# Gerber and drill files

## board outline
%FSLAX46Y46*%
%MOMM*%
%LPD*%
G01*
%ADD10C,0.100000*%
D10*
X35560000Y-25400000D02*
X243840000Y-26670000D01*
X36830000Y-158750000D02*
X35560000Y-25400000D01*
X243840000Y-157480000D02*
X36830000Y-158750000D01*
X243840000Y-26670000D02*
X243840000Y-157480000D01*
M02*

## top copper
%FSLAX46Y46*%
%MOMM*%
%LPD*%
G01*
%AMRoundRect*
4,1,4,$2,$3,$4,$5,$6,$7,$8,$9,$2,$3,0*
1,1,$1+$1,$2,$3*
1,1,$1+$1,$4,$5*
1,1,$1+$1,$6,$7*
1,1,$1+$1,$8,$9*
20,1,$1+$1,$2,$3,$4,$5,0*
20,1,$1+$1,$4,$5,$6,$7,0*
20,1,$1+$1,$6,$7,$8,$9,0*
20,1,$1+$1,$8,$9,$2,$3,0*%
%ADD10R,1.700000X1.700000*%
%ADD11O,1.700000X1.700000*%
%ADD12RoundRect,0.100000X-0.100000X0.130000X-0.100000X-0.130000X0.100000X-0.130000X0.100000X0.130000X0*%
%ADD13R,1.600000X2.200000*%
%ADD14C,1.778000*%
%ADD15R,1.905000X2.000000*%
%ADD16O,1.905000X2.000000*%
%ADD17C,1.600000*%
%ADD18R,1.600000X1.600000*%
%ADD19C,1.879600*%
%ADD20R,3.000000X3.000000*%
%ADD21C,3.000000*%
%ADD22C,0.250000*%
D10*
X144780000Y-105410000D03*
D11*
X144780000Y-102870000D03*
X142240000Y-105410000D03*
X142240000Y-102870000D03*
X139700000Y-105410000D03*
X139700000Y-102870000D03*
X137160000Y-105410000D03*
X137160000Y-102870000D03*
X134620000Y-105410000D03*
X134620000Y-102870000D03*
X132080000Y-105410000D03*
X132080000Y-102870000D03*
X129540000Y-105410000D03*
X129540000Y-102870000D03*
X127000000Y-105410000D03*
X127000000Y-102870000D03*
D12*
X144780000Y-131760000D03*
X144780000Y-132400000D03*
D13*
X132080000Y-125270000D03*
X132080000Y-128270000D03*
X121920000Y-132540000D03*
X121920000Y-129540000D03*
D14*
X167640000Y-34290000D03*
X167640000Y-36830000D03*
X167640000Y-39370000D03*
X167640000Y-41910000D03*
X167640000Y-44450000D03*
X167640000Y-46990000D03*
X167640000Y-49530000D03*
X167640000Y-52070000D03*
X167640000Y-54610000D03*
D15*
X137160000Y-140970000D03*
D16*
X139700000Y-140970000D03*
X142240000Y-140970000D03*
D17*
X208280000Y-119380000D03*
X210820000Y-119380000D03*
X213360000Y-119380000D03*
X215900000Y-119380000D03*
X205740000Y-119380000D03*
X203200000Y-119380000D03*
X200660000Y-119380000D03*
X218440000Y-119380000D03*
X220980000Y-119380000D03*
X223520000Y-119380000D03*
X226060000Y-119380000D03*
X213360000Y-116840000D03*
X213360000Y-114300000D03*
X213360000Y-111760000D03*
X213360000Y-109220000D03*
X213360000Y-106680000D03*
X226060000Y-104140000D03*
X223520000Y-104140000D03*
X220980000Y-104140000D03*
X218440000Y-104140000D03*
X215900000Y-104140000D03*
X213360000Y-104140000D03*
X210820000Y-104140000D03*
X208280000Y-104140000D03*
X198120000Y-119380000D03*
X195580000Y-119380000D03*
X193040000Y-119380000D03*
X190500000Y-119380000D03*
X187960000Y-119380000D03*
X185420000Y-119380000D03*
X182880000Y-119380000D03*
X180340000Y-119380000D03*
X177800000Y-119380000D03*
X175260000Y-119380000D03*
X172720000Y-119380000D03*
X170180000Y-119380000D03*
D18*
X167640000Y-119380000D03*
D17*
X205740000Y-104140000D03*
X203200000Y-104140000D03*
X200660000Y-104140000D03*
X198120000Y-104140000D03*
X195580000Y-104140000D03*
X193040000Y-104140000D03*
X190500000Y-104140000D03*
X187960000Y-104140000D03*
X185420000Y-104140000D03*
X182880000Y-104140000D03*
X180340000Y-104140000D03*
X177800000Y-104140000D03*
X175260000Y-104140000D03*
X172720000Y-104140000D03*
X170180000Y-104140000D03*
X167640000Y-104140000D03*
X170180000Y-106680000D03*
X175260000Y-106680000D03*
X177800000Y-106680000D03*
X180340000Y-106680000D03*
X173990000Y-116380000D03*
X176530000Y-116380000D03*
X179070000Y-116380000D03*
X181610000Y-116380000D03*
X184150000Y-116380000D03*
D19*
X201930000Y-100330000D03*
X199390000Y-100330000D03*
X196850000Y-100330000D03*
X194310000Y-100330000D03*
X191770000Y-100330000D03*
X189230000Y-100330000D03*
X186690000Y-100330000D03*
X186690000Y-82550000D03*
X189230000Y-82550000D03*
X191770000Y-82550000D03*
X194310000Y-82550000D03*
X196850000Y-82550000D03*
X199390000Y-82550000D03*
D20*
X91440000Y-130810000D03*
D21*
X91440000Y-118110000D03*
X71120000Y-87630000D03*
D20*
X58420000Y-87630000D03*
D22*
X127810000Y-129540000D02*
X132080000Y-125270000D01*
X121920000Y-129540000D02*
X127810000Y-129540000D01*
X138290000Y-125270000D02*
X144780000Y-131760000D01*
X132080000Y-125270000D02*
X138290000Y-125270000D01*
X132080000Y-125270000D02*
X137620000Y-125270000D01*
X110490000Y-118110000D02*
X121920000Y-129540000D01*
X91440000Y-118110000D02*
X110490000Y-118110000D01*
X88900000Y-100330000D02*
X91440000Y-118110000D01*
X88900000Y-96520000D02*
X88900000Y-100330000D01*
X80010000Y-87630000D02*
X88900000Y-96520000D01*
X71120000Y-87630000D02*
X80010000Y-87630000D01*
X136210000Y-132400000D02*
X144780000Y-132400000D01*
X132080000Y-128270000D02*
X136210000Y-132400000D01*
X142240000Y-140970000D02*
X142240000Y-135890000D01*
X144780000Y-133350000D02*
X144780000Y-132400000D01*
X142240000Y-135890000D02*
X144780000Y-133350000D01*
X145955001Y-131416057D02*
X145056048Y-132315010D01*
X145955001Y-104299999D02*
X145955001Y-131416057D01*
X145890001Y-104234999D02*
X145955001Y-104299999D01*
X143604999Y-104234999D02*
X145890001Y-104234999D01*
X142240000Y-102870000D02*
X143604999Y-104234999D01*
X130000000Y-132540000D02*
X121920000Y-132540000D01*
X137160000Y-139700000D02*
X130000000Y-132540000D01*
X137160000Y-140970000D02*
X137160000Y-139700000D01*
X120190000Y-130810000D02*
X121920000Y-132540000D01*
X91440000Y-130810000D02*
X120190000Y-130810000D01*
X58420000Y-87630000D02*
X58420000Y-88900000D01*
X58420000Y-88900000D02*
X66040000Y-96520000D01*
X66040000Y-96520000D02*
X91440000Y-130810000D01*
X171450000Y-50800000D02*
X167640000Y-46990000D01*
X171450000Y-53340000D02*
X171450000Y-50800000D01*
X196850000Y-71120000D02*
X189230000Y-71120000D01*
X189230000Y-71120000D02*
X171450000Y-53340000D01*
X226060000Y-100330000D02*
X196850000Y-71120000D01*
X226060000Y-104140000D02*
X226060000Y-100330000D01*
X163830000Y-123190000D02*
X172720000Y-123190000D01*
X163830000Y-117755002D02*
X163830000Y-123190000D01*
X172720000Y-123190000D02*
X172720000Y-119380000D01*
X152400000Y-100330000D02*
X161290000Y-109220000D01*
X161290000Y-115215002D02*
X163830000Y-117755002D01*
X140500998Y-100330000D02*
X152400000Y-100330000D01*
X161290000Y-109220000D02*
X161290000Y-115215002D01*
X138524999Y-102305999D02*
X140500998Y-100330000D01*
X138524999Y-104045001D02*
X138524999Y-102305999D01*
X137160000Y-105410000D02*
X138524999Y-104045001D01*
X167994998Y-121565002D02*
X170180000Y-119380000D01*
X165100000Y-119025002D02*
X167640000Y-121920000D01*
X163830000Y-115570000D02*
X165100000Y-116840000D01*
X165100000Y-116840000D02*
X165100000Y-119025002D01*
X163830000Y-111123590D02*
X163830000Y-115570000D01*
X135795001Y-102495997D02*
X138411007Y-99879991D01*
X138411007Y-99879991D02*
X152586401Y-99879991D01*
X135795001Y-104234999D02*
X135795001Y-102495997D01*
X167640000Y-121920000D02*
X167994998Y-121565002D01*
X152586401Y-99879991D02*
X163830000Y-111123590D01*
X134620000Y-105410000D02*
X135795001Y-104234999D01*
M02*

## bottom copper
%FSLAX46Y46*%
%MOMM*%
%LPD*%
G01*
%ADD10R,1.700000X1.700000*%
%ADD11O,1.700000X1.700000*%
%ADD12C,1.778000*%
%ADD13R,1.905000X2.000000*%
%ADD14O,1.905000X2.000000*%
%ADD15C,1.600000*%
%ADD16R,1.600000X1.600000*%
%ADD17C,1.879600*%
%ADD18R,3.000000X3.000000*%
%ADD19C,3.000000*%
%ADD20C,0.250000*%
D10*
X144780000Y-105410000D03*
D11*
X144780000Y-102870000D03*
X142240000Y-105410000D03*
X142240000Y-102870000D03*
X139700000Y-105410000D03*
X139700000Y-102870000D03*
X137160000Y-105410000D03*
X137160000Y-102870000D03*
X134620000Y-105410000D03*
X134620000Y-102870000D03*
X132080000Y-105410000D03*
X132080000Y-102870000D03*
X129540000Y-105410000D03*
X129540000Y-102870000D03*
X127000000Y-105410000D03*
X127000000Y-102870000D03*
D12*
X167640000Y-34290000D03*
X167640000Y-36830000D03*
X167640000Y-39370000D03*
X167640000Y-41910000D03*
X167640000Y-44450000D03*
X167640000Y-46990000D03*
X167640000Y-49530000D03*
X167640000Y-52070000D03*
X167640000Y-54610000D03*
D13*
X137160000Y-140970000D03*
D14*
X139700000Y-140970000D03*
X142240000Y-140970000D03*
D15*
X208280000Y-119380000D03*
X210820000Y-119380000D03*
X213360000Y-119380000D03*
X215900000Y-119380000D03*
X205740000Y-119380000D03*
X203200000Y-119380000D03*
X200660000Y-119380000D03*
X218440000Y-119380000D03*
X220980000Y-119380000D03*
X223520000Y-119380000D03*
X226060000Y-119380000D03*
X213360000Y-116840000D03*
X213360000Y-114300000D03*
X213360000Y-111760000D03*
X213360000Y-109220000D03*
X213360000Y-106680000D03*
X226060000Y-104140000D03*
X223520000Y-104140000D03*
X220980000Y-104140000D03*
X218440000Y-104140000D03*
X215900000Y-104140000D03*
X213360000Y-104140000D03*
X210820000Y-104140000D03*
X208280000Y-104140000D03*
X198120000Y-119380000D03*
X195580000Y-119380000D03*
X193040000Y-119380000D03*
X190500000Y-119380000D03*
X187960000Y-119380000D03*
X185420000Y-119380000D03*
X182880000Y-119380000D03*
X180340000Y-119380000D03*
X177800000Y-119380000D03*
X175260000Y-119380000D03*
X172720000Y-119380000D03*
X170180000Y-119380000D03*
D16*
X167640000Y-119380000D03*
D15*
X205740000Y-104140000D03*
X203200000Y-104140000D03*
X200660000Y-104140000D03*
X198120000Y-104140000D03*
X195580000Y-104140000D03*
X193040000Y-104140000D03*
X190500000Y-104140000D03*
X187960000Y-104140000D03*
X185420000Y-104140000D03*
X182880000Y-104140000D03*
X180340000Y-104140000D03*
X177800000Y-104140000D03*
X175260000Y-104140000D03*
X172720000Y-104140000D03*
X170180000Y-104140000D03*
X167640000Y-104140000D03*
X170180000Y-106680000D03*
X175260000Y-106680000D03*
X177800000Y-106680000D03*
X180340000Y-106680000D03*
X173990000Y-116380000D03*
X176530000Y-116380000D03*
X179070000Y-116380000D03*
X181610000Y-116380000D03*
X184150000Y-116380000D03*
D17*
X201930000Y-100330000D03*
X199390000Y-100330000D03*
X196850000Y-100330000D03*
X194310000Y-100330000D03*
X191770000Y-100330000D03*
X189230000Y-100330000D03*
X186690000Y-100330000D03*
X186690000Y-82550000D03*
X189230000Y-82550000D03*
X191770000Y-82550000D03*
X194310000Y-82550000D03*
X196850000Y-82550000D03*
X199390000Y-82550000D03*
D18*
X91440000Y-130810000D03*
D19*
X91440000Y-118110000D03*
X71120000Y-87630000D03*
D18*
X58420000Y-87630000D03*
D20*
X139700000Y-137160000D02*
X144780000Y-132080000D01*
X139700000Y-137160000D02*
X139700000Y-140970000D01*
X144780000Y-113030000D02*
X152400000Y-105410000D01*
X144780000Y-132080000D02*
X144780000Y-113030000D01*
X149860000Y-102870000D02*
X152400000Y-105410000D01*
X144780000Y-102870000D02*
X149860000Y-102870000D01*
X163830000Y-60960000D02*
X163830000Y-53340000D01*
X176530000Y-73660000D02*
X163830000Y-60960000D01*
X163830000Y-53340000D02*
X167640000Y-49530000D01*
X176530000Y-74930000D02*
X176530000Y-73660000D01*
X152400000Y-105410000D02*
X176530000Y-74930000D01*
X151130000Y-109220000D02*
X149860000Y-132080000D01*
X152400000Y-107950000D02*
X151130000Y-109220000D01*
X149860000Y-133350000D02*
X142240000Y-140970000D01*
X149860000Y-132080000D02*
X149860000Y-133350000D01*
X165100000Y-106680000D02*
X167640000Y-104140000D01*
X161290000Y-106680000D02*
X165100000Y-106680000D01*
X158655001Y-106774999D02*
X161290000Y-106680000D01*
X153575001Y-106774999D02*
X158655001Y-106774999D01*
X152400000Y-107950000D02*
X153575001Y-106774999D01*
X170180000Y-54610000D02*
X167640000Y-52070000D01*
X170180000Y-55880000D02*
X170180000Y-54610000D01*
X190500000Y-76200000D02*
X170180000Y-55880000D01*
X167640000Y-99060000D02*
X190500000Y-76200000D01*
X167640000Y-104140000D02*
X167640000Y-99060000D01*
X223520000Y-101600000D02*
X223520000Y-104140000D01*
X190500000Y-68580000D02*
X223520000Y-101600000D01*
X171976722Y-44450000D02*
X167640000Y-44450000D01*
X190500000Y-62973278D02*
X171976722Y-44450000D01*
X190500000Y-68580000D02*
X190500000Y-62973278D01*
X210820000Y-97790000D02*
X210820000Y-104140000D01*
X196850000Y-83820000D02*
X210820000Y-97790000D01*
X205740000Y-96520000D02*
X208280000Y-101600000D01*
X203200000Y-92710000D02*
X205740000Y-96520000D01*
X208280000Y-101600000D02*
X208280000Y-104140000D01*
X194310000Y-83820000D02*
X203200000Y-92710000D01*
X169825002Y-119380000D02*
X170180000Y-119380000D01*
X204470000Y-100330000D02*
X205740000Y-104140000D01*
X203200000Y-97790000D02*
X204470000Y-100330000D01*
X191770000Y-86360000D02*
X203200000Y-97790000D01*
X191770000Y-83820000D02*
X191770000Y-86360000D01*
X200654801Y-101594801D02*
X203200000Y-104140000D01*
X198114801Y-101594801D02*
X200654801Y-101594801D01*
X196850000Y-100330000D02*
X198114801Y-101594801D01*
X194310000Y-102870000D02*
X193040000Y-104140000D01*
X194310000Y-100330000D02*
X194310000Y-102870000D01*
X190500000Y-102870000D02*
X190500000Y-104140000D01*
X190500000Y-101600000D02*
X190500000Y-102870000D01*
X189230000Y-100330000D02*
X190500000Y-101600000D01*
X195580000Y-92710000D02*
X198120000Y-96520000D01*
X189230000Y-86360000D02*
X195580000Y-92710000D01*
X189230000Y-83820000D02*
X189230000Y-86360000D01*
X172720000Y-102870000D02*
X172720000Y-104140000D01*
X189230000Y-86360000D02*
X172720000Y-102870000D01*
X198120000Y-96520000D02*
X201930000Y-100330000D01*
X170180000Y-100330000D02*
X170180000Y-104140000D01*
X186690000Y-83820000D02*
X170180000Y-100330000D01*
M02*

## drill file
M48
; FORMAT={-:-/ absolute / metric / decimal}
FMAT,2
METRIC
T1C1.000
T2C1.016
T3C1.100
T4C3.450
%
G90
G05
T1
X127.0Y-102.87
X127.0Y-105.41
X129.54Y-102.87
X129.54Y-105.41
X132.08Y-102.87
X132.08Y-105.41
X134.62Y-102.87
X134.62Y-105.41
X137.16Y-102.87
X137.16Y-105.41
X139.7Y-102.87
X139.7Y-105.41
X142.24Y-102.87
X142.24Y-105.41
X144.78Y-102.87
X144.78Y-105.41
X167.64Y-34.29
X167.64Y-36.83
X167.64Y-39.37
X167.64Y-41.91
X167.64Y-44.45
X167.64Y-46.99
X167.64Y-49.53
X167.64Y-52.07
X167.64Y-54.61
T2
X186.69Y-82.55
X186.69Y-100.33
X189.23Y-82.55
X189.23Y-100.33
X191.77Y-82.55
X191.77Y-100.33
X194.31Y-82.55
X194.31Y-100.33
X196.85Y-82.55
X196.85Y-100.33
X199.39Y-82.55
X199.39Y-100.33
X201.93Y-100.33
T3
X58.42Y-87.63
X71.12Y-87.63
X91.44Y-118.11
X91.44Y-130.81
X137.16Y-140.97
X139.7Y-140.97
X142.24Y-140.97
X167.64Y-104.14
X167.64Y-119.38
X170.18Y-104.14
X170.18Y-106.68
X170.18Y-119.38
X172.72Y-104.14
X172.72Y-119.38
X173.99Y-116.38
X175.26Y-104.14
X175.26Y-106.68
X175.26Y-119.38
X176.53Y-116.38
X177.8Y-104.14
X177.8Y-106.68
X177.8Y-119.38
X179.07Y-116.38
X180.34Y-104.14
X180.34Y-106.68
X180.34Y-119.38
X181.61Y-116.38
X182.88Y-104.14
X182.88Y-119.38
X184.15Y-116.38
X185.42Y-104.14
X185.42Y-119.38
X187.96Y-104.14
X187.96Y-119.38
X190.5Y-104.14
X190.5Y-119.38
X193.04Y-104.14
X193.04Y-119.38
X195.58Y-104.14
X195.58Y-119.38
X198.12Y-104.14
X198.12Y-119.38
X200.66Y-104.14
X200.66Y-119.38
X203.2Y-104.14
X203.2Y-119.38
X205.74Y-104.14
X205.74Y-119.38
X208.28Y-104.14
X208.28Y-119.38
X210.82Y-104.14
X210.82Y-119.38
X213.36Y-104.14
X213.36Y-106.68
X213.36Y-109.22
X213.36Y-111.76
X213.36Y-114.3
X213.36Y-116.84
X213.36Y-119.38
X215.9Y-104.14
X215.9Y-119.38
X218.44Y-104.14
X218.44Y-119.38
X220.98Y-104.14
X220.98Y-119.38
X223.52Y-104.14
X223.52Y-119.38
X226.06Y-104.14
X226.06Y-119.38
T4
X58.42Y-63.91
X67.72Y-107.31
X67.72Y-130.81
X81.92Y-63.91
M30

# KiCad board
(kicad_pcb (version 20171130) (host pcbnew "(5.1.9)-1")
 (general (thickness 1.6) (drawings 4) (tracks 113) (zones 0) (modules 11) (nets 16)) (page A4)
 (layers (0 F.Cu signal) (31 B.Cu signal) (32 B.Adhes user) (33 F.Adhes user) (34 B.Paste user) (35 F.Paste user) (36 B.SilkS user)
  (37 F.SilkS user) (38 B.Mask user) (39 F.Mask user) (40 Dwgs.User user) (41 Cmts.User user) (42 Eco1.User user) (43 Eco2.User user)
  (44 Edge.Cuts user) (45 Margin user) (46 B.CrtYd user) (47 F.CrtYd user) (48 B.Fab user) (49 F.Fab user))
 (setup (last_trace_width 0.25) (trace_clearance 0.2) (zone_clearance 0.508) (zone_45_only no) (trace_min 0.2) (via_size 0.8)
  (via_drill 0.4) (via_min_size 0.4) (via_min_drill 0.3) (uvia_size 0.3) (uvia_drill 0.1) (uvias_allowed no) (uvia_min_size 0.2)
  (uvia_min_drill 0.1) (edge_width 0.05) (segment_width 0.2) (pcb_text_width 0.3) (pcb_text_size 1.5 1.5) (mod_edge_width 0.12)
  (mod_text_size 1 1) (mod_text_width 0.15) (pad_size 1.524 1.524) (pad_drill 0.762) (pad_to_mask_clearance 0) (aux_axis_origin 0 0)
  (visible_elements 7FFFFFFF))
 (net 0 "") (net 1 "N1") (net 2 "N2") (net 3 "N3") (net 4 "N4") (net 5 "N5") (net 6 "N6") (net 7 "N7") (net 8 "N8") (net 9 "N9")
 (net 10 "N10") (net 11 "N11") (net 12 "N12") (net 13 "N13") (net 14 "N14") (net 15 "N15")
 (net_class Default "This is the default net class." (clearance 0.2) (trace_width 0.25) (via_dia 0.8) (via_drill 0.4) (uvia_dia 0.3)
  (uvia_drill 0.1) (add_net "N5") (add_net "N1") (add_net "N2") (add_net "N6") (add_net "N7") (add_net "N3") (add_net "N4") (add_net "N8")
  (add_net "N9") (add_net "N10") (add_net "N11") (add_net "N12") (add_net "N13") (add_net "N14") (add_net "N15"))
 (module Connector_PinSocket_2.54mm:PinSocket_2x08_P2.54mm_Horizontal (layer F.Cu) (at 144.78 105.41 270)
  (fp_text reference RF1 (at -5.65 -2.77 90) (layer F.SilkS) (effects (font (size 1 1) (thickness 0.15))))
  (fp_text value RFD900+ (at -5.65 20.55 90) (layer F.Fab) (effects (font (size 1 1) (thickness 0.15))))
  (pad 1 thru_hole rect (at 0 0 270) (size 1.7 1.7) (drill 1) (layers *.Cu *.Mask))
  (pad 2 thru_hole oval (at -2.54 0 270) (size 1.7 1.7) (drill 1) (layers *.Cu *.Mask) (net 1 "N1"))
  (pad 3 thru_hole oval (at 0 2.54 270) (size 1.7 1.7) (drill 1) (layers *.Cu *.Mask))
  (pad 4 thru_hole oval (at -2.54 2.54 270) (size 1.7 1.7) (drill 1) (layers *.Cu *.Mask) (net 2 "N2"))
  (pad 5 thru_hole oval (at 0 5.08 270) (size 1.7 1.7) (drill 1) (layers *.Cu *.Mask))
  (pad 6 thru_hole oval (at -2.54 5.08 270) (size 1.7 1.7) (drill 1) (layers *.Cu *.Mask))
  (pad 7 thru_hole oval (at 0 7.62 270) (size 1.7 1.7) (drill 1) (layers *.Cu *.Mask) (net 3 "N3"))
  (pad 8 thru_hole oval (at -2.54 7.62 270) (size 1.7 1.7) (drill 1) (layers *.Cu *.Mask))
  (pad 9 thru_hole oval (at 0 10.16 270) (size 1.7 1.7) (drill 1) (layers *.Cu *.Mask) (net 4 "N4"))
  (pad 10 thru_hole oval (at -2.54 10.16 270) (size 1.7 1.7) (drill 1) (layers *.Cu *.Mask))
  (pad 11 thru_hole oval (at 0 12.7 270) (size 1.7 1.7) (drill 1) (layers *.Cu *.Mask))
  (pad 12 thru_hole oval (at -2.54 12.7 270) (size 1.7 1.7) (drill 1) (layers *.Cu *.Mask))
  (pad 13 thru_hole oval (at 0 15.24 270) (size 1.7 1.7) (drill 1) (layers *.Cu *.Mask))
  (pad 14 thru_hole oval (at -2.54 15.24 270) (size 1.7 1.7) (drill 1) (layers *.Cu *.Mask))
  (pad 15 thru_hole oval (at 0 17.78 270) (size 1.7 1.7) (drill 1) (layers *.Cu *.Mask))
  (pad 16 thru_hole oval (at -2.54 17.78 270) (size 1.7 1.7) (drill 1) (layers *.Cu *.Mask)))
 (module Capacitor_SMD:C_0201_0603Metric (layer F.Cu) (at 144.78 132.08 270)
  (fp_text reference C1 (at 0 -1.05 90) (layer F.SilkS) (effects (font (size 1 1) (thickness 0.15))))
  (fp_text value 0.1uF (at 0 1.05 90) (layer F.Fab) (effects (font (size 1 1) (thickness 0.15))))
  (pad "" smd roundrect (at -0.345 0 270) (size 0.318 0.36) (layers F.Paste) (roundrect_rratio 0.25))
  (pad "" smd roundrect (at 0.345 0 270) (size 0.318 0.36) (layers F.Paste) (roundrect_rratio 0.25))
  (pad 1 smd roundrect (at -0.32 0 270) (size 0.46 0.4) (layers F.Cu F.Mask) (roundrect_rratio 0.25) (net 1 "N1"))
  (pad 2 smd roundrect (at 0.32 0 270) (size 0.46 0.4) (layers F.Cu F.Mask) (roundrect_rratio 0.25) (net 2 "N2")))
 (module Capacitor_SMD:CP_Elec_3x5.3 (layer F.Cu) (at 132.08 126.77 90)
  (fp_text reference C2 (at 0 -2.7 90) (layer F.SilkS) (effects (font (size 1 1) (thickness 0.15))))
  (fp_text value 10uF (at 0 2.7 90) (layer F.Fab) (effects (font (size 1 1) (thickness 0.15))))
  (pad 2 smd rect (at 1.5 0 90) (size 2.2 1.6) (layers F.Cu F.Paste F.Mask) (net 1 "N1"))
  (pad 1 smd rect (at -1.5 0 90) (size 2.2 1.6) (layers F.Cu F.Paste F.Mask) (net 2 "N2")))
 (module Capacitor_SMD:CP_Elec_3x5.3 (layer F.Cu) (at 121.92 131.04 90)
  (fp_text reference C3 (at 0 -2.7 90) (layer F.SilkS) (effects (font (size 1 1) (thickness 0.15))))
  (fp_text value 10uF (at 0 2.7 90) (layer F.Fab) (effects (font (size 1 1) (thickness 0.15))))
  (pad 1 smd rect (at -1.5 0 90) (size 2.2 1.6) (layers F.Cu F.Paste F.Mask) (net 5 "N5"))
  (pad 2 smd rect (at 1.5 0 90) (size 2.2 1.6) (layers F.Cu F.Paste F.Mask) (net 1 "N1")))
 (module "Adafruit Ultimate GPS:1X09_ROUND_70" (layer F.Cu) (at 167.64 44.45 270)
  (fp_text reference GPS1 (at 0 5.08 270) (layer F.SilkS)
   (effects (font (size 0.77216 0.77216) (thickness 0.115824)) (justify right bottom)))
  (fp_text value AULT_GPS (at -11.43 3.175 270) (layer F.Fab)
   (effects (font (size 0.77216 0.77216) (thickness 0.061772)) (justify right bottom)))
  (pad 1 thru_hole circle (at -10.16 0) (size 1.778 1.778) (drill 1) (layers *.Cu *.Mask) (solder_mask_margin 0.0508))
  (pad 2 thru_hole circle (at -7.62 0) (size 1.778 1.778) (drill 1) (layers *.Cu *.Mask) (solder_mask_margin 0.0508))
  (pad 3 thru_hole circle (at -5.08 0) (size 1.778 1.778) (drill 1) (layers *.Cu *.Mask) (solder_mask_margin 0.0508))
  (pad 4 thru_hole circle (at -2.54 0) (size 1.778 1.778) (drill 1) (layers *.Cu *.Mask) (solder_mask_margin 0.0508))
  (pad 5 thru_hole circle (at 0 0) (size 1.778 1.778) (drill 1) (layers *.Cu *.Mask) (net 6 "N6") (solder_mask_margin 0.0508))
  (pad 6 thru_hole circle (at 2.54 0) (size 1.778 1.778) (drill 1) (layers *.Cu *.Mask) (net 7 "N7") (solder_mask_margin 0.0508))
  (pad 7 thru_hole circle (at 5.08 0) (size 1.778 1.778) (drill 1) (layers *.Cu *.Mask) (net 1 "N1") (solder_mask_margin 0.0508))
  (pad 8 thru_hole circle (at 7.62 0) (size 1.778 1.778) (drill 1) (layers *.Cu *.Mask) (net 2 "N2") (solder_mask_margin 0.0508))
  (pad 9 thru_hole circle (at 10.16 0) (size 1.778 1.778) (drill 1) (layers *.Cu *.Mask) (solder_mask_margin 0.0508)))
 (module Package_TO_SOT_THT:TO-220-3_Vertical (layer F.Cu) (at 137.16 140.97)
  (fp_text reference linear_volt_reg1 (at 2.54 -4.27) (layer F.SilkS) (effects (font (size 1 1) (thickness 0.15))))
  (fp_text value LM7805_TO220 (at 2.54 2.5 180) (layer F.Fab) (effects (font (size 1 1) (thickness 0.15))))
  (pad 1 thru_hole rect (at 0 0) (size 1.905 2) (drill 1.1) (layers *.Cu *.Mask) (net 5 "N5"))
  (pad 2 thru_hole oval (at 2.54 0) (size 1.905 2) (drill 1.1) (layers *.Cu *.Mask) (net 1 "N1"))
  (pad 3 thru_hole oval (at 5.08 0) (size 1.905 2) (drill 1.1) (layers *.Cu *.Mask) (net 2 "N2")))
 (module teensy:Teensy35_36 (layer F.Cu) (at 196.85 111.76)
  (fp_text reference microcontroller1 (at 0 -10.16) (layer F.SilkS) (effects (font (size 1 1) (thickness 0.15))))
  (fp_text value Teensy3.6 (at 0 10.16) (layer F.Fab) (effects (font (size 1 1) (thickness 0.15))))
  (pad 17 thru_hole circle (at 11.43 7.62) (size 1.6 1.6) (drill 1.1) (layers *.Cu *.Mask))
  (pad 18 thru_hole circle (at 13.97 7.62) (size 1.6 1.6) (drill 1.1) (layers *.Cu *.Mask))
  (pad 19 thru_hole circle (at 16.51 7.62) (size 1.6 1.6) (drill 1.1) (layers *.Cu *.Mask))
  (pad 20 thru_hole circle (at 19.05 7.62) (size 1.6 1.6) (drill 1.1) (layers *.Cu *.Mask))
  (pad 16 thru_hole circle (at 8.89 7.62) (size 1.6 1.6) (drill 1.1) (layers *.Cu *.Mask))
  (pad 15 thru_hole circle (at 6.35 7.62) (size 1.6 1.6) (drill 1.1) (layers *.Cu *.Mask))
  (pad 14 thru_hole circle (at 3.81 7.62) (size 1.6 1.6) (drill 1.1) (layers *.Cu *.Mask))
  (pad 21 thru_hole circle (at 21.59 7.62) (size 1.6 1.6) (drill 1.1) (layers *.Cu *.Mask))
  (pad 22 thru_hole circle (at 24.13 7.62) (size 1.6 1.6) (drill 1.1) (layers *.Cu *.Mask))
  (pad 23 thru_hole circle (at 26.67 7.62) (size 1.6 1.6) (drill 1.1) (layers *.Cu *.Mask))
  (pad 24 thru_hole circle (at 29.21 7.62) (size 1.6 1.6) (drill 1.1) (layers *.Cu *.Mask))
  (pad 25 thru_hole circle (at 16.51 5.08) (size 1.6 1.6) (drill 1.1) (layers *.Cu *.Mask))
  (pad 26 thru_hole circle (at 16.51 2.54) (size 1.6 1.6) (drill 1.1) (layers *.Cu *.Mask))
  (pad 27 thru_hole circle (at 16.51 0) (size 1.6 1.6) (drill 1.1) (layers *.Cu *.Mask))
  (pad 28 thru_hole circle (at 16.51 -2.54) (size 1.6 1.6) (drill 1.1) (layers *.Cu *.Mask))
  (pad 29 thru_hole circle (at 16.51 -5.08) (size 1.6 1.6) (drill 1.1) (layers *.Cu *.Mask))
  (pad 30 thru_hole circle (at 29.21 -7.62) (size 1.6 1.6) (drill 1.1) (layers *.Cu *.Mask) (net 7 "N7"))
  (pad 31 thru_hole circle (at 26.67 -7.62) (size 1.6 1.6) (drill 1.1) (layers *.Cu *.Mask) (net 6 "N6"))
  (pad 32 thru_hole circle (at 24.13 -7.62) (size 1.6 1.6) (drill 1.1) (layers *.Cu *.Mask))
  (pad 33 thru_hole circle (at 21.59 -7.62) (size 1.6 1.6) (drill 1.1) (layers *.Cu *.Mask))
  (pad 34 thru_hole circle (at 19.05 -7.62) (size 1.6 1.6) (drill 1.1) (layers *.Cu *.Mask))
  (pad 35 thru_hole circle (at 16.51 -7.62) (size 1.6 1.6) (drill 1.1) (layers *.Cu *.Mask))
  (pad 36 thru_hole circle (at 13.97 -7.62) (size 1.6 1.6) (drill 1.1) (layers *.Cu *.Mask) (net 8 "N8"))
  (pad 37 thru_hole circle (at 11.43 -7.62) (size 1.6 1.6) (drill 1.1) (layers *.Cu *.Mask) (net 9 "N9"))
  (pad 13 thru_hole circle (at 1.27 7.62) (size 1.6 1.6) (drill 1.1) (layers *.Cu *.Mask))
  (pad 12 thru_hole circle (at -1.27 7.62) (size 1.6 1.6) (drill 1.1) (layers *.Cu *.Mask))
  (pad 11 thru_hole circle (at -3.81 7.62) (size 1.6 1.6) (drill 1.1) (layers *.Cu *.Mask))
  (pad 10 thru_hole circle (at -6.35 7.62) (size 1.6 1.6) (drill 1.1) (layers *.Cu *.Mask))
  (pad 9 thru_hole circle (at -8.89 7.62) (size 1.6 1.6) (drill 1.1) (layers *.Cu *.Mask))
  (pad 8 thru_hole circle (at -11.43 7.62) (size 1.6 1.6) (drill 1.1) (layers *.Cu *.Mask))
  (pad 7 thru_hole circle (at -13.97 7.62) (size 1.6 1.6) (drill 1.1) (layers *.Cu *.Mask))
  (pad 6 thru_hole circle (at -16.51 7.62) (size 1.6 1.6) (drill 1.1) (layers *.Cu *.Mask))
  (pad 5 thru_hole circle (at -19.05 7.62) (size 1.6 1.6) (drill 1.1) (layers *.Cu *.Mask))
  (pad 4 thru_hole circle (at -21.59 7.62) (size 1.6 1.6) (drill 1.1) (layers *.Cu *.Mask))
  (pad 3 thru_hole circle (at -24.13 7.62) (size 1.6 1.6) (drill 1.1) (layers *.Cu *.Mask) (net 3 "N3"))
  (pad 2 thru_hole circle (at -26.67 7.62) (size 1.6 1.6) (drill 1.1) (layers *.Cu *.Mask) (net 4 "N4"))
  (pad 1 thru_hole rect (at -29.21 7.62) (size 1.6 1.6) (drill 1.1) (layers *.Cu *.Mask))
  (pad 38 thru_hole circle (at 8.89 -7.62) (size 1.6 1.6) (drill 1.1) (layers *.Cu *.Mask) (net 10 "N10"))
  (pad 39 thru_hole circle (at 6.35 -7.62) (size 1.6 1.6) (drill 1.1) (layers *.Cu *.Mask) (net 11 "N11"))
  (pad 40 thru_hole circle (at 3.81 -7.62) (size 1.6 1.6) (drill 1.1) (layers *.Cu *.Mask))
  (pad 41 thru_hole circle (at 1.27 -7.62) (size 1.6 1.6) (drill 1.1) (layers *.Cu *.Mask))
  (pad 42 thru_hole circle (at -1.27 -7.62) (size 1.6 1.6) (drill 1.1) (layers *.Cu *.Mask))
  (pad 43 thru_hole circle (at -3.81 -7.62) (size 1.6 1.6) (drill 1.1) (layers *.Cu *.Mask) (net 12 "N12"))
  (pad 44 thru_hole circle (at -6.35 -7.62) (size 1.6 1.6) (drill 1.1) (layers *.Cu *.Mask) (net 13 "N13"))
  (pad 45 thru_hole circle (at -8.89 -7.62) (size 1.6 1.6) (drill 1.1) (layers *.Cu *.Mask))
  (pad 46 thru_hole circle (at -11.43 -7.62) (size 1.6 1.6) (drill 1.1) (layers *.Cu *.Mask))
  (pad 47 thru_hole circle (at -13.97 -7.62) (size 1.6 1.6) (drill 1.1) (layers *.Cu *.Mask))
  (pad 48 thru_hole circle (at -16.51 -7.62) (size 1.6 1.6) (drill 1.1) (layers *.Cu *.Mask))
  (pad 49 thru_hole circle (at -19.05 -7.62) (size 1.6 1.6) (drill 1.1) (layers *.Cu *.Mask))
  (pad 50 thru_hole circle (at -21.59 -7.62) (size 1.6 1.6) (drill 1.1) (layers *.Cu *.Mask))
  (pad 51 thru_hole circle (at -24.13 -7.62) (size 1.6 1.6) (drill 1.1) (layers *.Cu *.Mask) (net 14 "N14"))
  (pad 52 thru_hole circle (at -26.67 -7.62) (size 1.6 1.6) (drill 1.1) (layers *.Cu *.Mask) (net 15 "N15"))
  (pad 53 thru_hole circle (at -29.21 -7.62) (size 1.6 1.6) (drill 1.1) (layers *.Cu *.Mask) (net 2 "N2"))
  (pad 54 thru_hole circle (at -26.67 -5.08) (size 1.6 1.6) (drill 1.1) (layers *.Cu *.Mask))
  (pad 55 thru_hole circle (at -21.59 -5.08) (size 1.6 1.6) (drill 1.1) (layers *.Cu *.Mask))
  (pad 56 thru_hole circle (at -19.05 -5.08) (size 1.6 1.6) (drill 1.1) (layers *.Cu *.Mask))
  (pad 57 thru_hole circle (at -16.51 -5.08) (size 1.6 1.6) (drill 1.1) (layers *.Cu *.Mask))
  (pad 58 thru_hole circle (at -22.86 4.62) (size 1.6 1.6) (drill 1.1) (layers *.Cu *.Mask))
  (pad 59 thru_hole circle (at -20.32 4.62) (size 1.6 1.6) (drill 1.1) (layers *.Cu *.Mask))
  (pad 60 thru_hole circle (at -17.78 4.62) (size 1.6 1.6) (drill 1.1) (layers *.Cu *.Mask))
  (pad 61 thru_hole circle (at -15.24 4.62) (size 1.6 1.6) (drill 1.1) (layers *.Cu *.Mask))
  (pad 62 thru_hole circle (at -12.7 4.62) (size 1.6 1.6) (drill 1.1) (layers *.Cu *.Mask)))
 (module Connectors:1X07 (layer F.Cu) (at 201.93 100.33 180)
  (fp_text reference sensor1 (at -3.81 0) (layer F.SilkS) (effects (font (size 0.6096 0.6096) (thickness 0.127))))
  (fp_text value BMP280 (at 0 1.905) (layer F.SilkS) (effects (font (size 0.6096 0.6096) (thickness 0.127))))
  (pad 1 thru_hole circle (at 0 0 180) (size 1.8796 1.8796) (drill 1.016) (layers *.Cu *.Mask) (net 14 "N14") (solder_mask_margin 0.1016))
  (pad 2 thru_hole circle (at 2.54 0 180) (size 1.8796 1.8796) (drill 1.016) (layers *.Cu *.Mask) (solder_mask_margin 0.1016))
  (pad 3 thru_hole circle (at 5.08 0 180) (size 1.8796 1.8796) (drill 1.016) (layers *.Cu *.Mask) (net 11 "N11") (solder_mask_margin 0.1016))
  (pad 4 thru_hole circle (at 7.62 0 180) (size 1.8796 1.8796) (drill 1.016) (layers *.Cu *.Mask) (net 12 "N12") (solder_mask_margin 0.1016))
  (pad 5 thru_hole circle (at 10.16 0 180) (size 1.8796 1.8796) (drill 1.016) (layers *.Cu *.Mask) (solder_mask_margin 0.1016))
  (pad 6 thru_hole circle (at 12.7 0 180) (size 1.8796 1.8796) (drill 1.016) (layers *.Cu *.Mask) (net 13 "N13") (solder_mask_margin 0.1016))
  (pad 7 thru_hole circle (at 15.24 0 180) (size 1.8796 1.8796) (drill 1.016) (layers *.Cu *.Mask) (solder_mask_margin 0.1016)))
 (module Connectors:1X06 (layer F.Cu) (at 186.69 82.55)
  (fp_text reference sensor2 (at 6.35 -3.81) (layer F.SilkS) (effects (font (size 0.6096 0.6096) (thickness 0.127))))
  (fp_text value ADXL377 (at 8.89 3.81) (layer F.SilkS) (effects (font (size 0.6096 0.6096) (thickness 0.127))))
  (pad 1 thru_hole circle (at 0 0) (size 1.8796 1.8796) (drill 1.016) (layers *.Cu *.Mask) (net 15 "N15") (solder_mask_margin 0.1016))
  (pad 2 thru_hole circle (at 2.54 0) (size 1.8796 1.8796) (drill 1.016) (layers *.Cu *.Mask) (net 14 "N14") (solder_mask_margin 0.1016))
  (pad 3 thru_hole circle (at 5.08 0) (size 1.8796 1.8796) (drill 1.016) (layers *.Cu *.Mask) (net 10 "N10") (solder_mask_margin 0.1016))
  (pad 4 thru_hole circle (at 7.62 0) (size 1.8796 1.8796) (drill 1.016) (layers *.Cu *.Mask) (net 9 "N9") (solder_mask_margin 0.1016))
  (pad 5 thru_hole circle (at 10.16 0) (size 1.8796 1.8796) (drill 1.016) (layers *.Cu *.Mask) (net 8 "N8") (solder_mask_margin 0.1016))
  (pad 6 thru_hole circle (at 12.7 0) (size 1.8796 1.8796) (drill 1.016) (layers *.Cu *.Mask) (solder_mask_margin 0.1016)))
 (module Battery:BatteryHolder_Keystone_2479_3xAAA (layer F.Cu) (at 91.44 130.81 180)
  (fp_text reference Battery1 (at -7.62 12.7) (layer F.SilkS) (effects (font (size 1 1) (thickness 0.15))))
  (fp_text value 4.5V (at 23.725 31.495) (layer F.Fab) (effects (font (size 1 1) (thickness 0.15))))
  (pad 1 thru_hole rect (at 0 0 180) (size 3 3) (drill 1.1) (layers *.Cu *.Mask) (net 5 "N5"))
  (pad 2 thru_hole circle (at 0 12.7 180) (size 3 3) (drill 1.1) (layers *.Cu *.Mask) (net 1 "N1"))
  (pad "" np_thru_hole circle (at 23.72 0 180) (size 3.45 3.45) (drill 3.45) (layers *.Cu *.Mask))
  (pad "" np_thru_hole circle (at 23.72 23.5 180) (size 3.45 3.45) (drill 3.45) (layers *.Cu *.Mask)))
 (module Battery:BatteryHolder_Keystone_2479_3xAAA (layer F.Cu) (at 58.42 87.63 90)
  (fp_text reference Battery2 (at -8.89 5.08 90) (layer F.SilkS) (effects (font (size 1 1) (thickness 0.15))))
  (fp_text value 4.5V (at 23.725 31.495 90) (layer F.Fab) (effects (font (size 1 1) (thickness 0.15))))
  (pad "" np_thru_hole circle (at 23.72 23.5 90) (size 3.45 3.45) (drill 3.45) (layers *.Cu *.Mask))
  (pad "" np_thru_hole circle (at 23.72 0 90) (size 3.45 3.45) (drill 3.45) (layers *.Cu *.Mask))
  (pad 2 thru_hole circle (at 0 12.7 90) (size 3 3) (drill 1.1) (layers *.Cu *.Mask) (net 1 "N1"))
  (pad 1 thru_hole rect (at 0 0 90) (size 3 3) (drill 1.1) (layers *.Cu *.Mask) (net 5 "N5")))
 (gr_line (start 35.56 25.4) (end 243.84 26.67) (layer Edge.Cuts) (width 0.1))
 (gr_line (start 36.83 158.75) (end 35.56 25.4) (layer Edge.Cuts) (width 0.1))
 (gr_line (start 243.84 157.48) (end 36.83 158.75) (layer Edge.Cuts) (width 0.1))
 (gr_line (start 243.84 26.67) (end 243.84 157.48) (layer Edge.Cuts) (width 0.1))
 (segment (start 127.81 129.54) (end 132.08 125.27) (width 0.25) (layer F.Cu) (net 1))
 (segment (start 121.92 129.54) (end 127.81 129.54) (width 0.25) (layer F.Cu) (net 1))
 (segment (start 138.29 125.27) (end 144.78 131.76) (width 0.25) (layer F.Cu) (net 1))
 (segment (start 132.08 125.27) (end 138.29 125.27) (width 0.25) (layer F.Cu) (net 1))
 (segment (start 139.7 137.16) (end 144.78 132.08) (width 0.25) (layer B.Cu) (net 1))
 (segment (start 139.7 137.16) (end 139.7 140.97) (width 0.25) (layer B.Cu) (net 1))
 (segment (start 132.08 125.27) (end 137.62 125.27) (width 0.25) (layer F.Cu) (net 1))
 (segment (start 144.78 113.03) (end 152.4 105.41) (width 0.25) (layer B.Cu) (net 1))
 (segment (start 144.78 132.08) (end 144.78 113.03) (width 0.25) (layer B.Cu) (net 1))
 (segment (start 110.49 118.11) (end 121.92 129.54) (width 0.25) (layer F.Cu) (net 1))
 (segment (start 91.44 118.11) (end 110.49 118.11) (width 0.25) (layer F.Cu) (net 1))
 (segment (start 88.9 100.33) (end 91.44 118.11) (width 0.25) (layer F.Cu) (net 1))
 (segment (start 88.9 96.52) (end 88.9 100.33) (width 0.25) (layer F.Cu) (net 1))
 (segment (start 80.01 87.63) (end 88.9 96.52) (width 0.25) (layer F.Cu) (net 1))
 (segment (start 71.12 87.63) (end 80.01 87.63) (width 0.25) (layer F.Cu) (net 1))
 (segment (start 149.86 102.87) (end 152.4 105.41) (width 0.25) (layer B.Cu) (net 1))
 (segment (start 144.78 102.87) (end 149.86 102.87) (width 0.25) (layer B.Cu) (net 1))
 (segment (start 163.83 60.96) (end 163.83 53.34) (width 0.25) (layer B.Cu) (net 1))
 (segment (start 176.53 73.66) (end 163.83 60.96) (width 0.25) (layer B.Cu) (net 1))
 (segment (start 163.83 53.34) (end 167.64 49.53) (width 0.25) (layer B.Cu) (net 1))
 (segment (start 176.53 74.93) (end 176.53 73.66) (width 0.25) (layer B.Cu) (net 1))
 (segment (start 152.4 105.41) (end 176.53 74.93) (width 0.25) (layer B.Cu) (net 1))
 (segment (start 136.21 132.4) (end 144.78 132.4) (width 0.25) (layer F.Cu) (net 2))
 (segment (start 132.08 128.27) (end 136.21 132.4) (width 0.25) (layer F.Cu) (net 2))
 (segment (start 142.24 140.97) (end 142.24 135.89) (width 0.25) (layer F.Cu) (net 2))
 (segment (start 144.78 133.35) (end 144.78 132.4) (width 0.25) (layer F.Cu) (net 2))
 (segment (start 142.24 135.89) (end 144.78 133.35) (width 0.25) (layer F.Cu) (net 2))
 (segment (start 151.13 109.22) (end 149.86 132.08) (width 0.25) (layer B.Cu) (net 2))
 (segment (start 152.4 107.95) (end 151.13 109.22) (width 0.25) (layer B.Cu) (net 2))
 (segment (start 149.86 133.35) (end 142.24 140.97) (width 0.25) (layer B.Cu) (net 2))
 (segment (start 149.86 132.08) (end 149.86 133.35) (width 0.25) (layer B.Cu) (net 2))
 (segment (start 165.1 106.68) (end 167.64 104.14) (width 0.25) (layer B.Cu) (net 2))
 (segment (start 161.29 106.68) (end 165.1 106.68) (width 0.25) (layer B.Cu) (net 2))
 (segment (start 158.655001 106.774999) (end 161.29 106.68) (width 0.25) (layer B.Cu) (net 2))
 (segment (start 153.575001 106.774999) (end 158.655001 106.774999) (width 0.25) (layer B.Cu) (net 2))
 (segment (start 152.4 107.95) (end 153.575001 106.774999) (width 0.25) (layer B.Cu) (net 2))
 (segment (start 145.955001 131.416057) (end 145.056048 132.31501) (width 0.25) (layer F.Cu) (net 2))
 (segment (start 145.955001 104.299999) (end 145.955001 131.416057) (width 0.25) (layer F.Cu) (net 2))
 (segment (start 145.890001 104.234999) (end 145.955001 104.299999) (width 0.25) (layer F.Cu) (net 2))
 (segment (start 143.604999 104.234999) (end 145.890001 104.234999) (width 0.25) (layer F.Cu) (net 2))
 (segment (start 142.24 102.87) (end 143.604999 104.234999) (width 0.25) (layer F.Cu) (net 2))
 (segment (start 170.18 54.61) (end 167.64 52.07) (width 0.25) (layer B.Cu) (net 2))
 (segment (start 170.18 55.88) (end 170.18 54.61) (width 0.25) (layer B.Cu) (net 2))
 (segment (start 190.5 76.2) (end 170.18 55.88) (width 0.25) (layer B.Cu) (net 2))
 (segment (start 167.64 99.06) (end 190.5 76.2) (width 0.25) (layer B.Cu) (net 2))
 (segment (start 167.64 104.14) (end 167.64 99.06) (width 0.25) (layer B.Cu) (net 2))
 (segment (start 130 132.54) (end 121.92 132.54) (width 0.25) (layer F.Cu) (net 5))
 (segment (start 137.16 139.7) (end 130 132.54) (width 0.25) (layer F.Cu) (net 5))
 (segment (start 137.16 140.97) (end 137.16 139.7) (width 0.25) (layer F.Cu) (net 5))
 (segment (start 120.19 130.81) (end 121.92 132.54) (width 0.25) (layer F.Cu) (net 5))
 (segment (start 91.44 130.81) (end 120.19 130.81) (width 0.25) (layer F.Cu) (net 5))
 (segment (start 58.42 87.63) (end 58.42 88.9) (width 0.25) (layer F.Cu) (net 5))
 (segment (start 58.42 88.9) (end 66.04 96.52) (width 0.25) (layer F.Cu) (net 5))
 (segment (start 66.04 96.52) (end 91.44 130.81) (width 0.25) (layer F.Cu) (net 5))
 (segment (start 223.52 101.6) (end 223.52 104.14) (width 0.25) (layer B.Cu) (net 6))
 (segment (start 190.5 68.58) (end 223.52 101.6) (width 0.25) (layer B.Cu) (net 6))
 (segment (start 171.976722 44.45) (end 167.64 44.45) (width 0.25) (layer B.Cu) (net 6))
 (segment (start 190.5 62.973278) (end 171.976722 44.45) (width 0.25) (layer B.Cu) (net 6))
 (segment (start 190.5 68.58) (end 190.5 62.973278) (width 0.25) (layer B.Cu) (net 6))
 (segment (start 171.45 50.8) (end 167.64 46.99) (width 0.25) (layer F.Cu) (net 7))
 (segment (start 171.45 53.34) (end 171.45 50.8) (width 0.25) (layer F.Cu) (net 7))
 (segment (start 196.85 71.12) (end 189.23 71.12) (width 0.25) (layer F.Cu) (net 7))
 (segment (start 189.23 71.12) (end 171.45 53.34) (width 0.25) (layer F.Cu) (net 7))
 (segment (start 226.06 100.33) (end 196.85 71.12) (width 0.25) (layer F.Cu) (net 7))
 (segment (start 226.06 104.14) (end 226.06 100.33) (width 0.25) (layer F.Cu) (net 7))
 (segment (start 210.82 97.79) (end 210.82 104.14) (width 0.25) (layer B.Cu) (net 8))
 (segment (start 196.85 83.82) (end 210.82 97.79) (width 0.25) (layer B.Cu) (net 8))
 (segment (start 205.74 96.52) (end 208.28 101.6) (width 0.25) (layer B.Cu) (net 9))
 (segment (start 203.2 92.71) (end 205.74 96.52) (width 0.25) (layer B.Cu) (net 9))
 (segment (start 208.28 101.6) (end 208.28 104.14) (width 0.25) (layer B.Cu) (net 9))
 (segment (start 194.31 83.82) (end 203.2 92.71) (width 0.25) (layer B.Cu) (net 9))
 (segment (start 163.83 123.19) (end 172.72 123.19) (width 0.25) (layer F.Cu) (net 3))
 (segment (start 163.83 117.755002) (end 163.83 123.19) (width 0.25) (layer F.Cu) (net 3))
 (segment (start 172.72 123.19) (end 172.72 119.38) (width 0.25) (layer F.Cu) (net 3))
 (segment (start 152.4 100.33) (end 161.29 109.22) (width 0.25) (layer F.Cu) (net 3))
 (segment (start 161.29 115.215002) (end 163.83 117.755002) (width 0.25) (layer F.Cu) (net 3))
 (segment (start 140.500998 100.33) (end 152.4 100.33) (width 0.25) (layer F.Cu) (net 3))
 (segment (start 161.29 109.22) (end 161.29 115.215002) (width 0.25) (layer F.Cu) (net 3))
 (segment (start 138.524999 102.305999) (end 140.500998 100.33) (width 0.25) (layer F.Cu) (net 3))
 (segment (start 138.524999 104.045001) (end 138.524999 102.305999) (width 0.25) (layer F.Cu) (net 3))
 (segment (start 137.16 105.41) (end 138.524999 104.045001) (width 0.25) (layer F.Cu) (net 3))
 (segment (start 169.825002 119.38) (end 170.18 119.38) (width 0.25) (layer B.Cu) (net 4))
 (segment (start 167.994998 121.565002) (end 170.18 119.38) (width 0.25) (layer F.Cu) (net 4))
 (segment (start 165.1 119.025002) (end 167.64 121.92) (width 0.25) (layer F.Cu) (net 4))
 (segment (start 163.83 115.57) (end 165.1 116.84) (width 0.25) (layer F.Cu) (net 4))
 (segment (start 165.1 116.84) (end 165.1 119.025002) (width 0.25) (layer F.Cu) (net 4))
 (segment (start 163.83 111.12359) (end 163.83 115.57) (width 0.25) (layer F.Cu) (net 4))
 (segment (start 135.795001 102.495997) (end 138.411007 99.879991) (width 0.25) (layer F.Cu) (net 4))
 (segment (start 138.411007 99.879991) (end 152.586401 99.879991) (width 0.25) (layer F.Cu) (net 4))
 (segment (start 135.795001 104.234999) (end 135.795001 102.495997) (width 0.25) (layer F.Cu) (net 4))
 (segment (start 167.64 121.92) (end 167.994998 121.565002) (width 0.25) (layer F.Cu) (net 4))
 (segment (start 152.586401 99.879991) (end 163.83 111.12359) (width 0.25) (layer F.Cu) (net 4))
 (segment (start 134.62 105.41) (end 135.795001 104.234999) (width 0.25) (layer F.Cu) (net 4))
 (segment (start 204.47 100.33) (end 205.74 104.14) (width 0.25) (layer B.Cu) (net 10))
 (segment (start 203.2 97.79) (end 204.47 100.33) (width 0.25) (layer B.Cu) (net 10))
 (segment (start 191.77 86.36) (end 203.2 97.79) (width 0.25) (layer B.Cu) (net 10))
 (segment (start 191.77 83.82) (end 191.77 86.36) (width 0.25) (layer B.Cu) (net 10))
 (segment (start 200.654801 101.594801) (end 203.2 104.14) (width 0.25) (layer B.Cu) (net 11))
 (segment (start 198.114801 101.594801) (end 200.654801 101.594801) (width 0.25) (layer B.Cu) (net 11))
 (segment (start 196.85 100.33) (end 198.114801 101.594801) (width 0.25) (layer B.Cu) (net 11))
 (segment (start 194.31 102.87) (end 193.04 104.14) (width 0.25) (layer B.Cu) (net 12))
 (segment (start 194.31 100.33) (end 194.31 102.87) (width 0.25) (layer B.Cu) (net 12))
 (segment (start 190.5 102.87) (end 190.5 104.14) (width 0.25) (layer B.Cu) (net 13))
 (segment (start 190.5 101.6) (end 190.5 102.87) (width 0.25) (layer B.Cu) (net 13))
 (segment (start 189.23 100.33) (end 190.5 101.6) (width 0.25) (layer B.Cu) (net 13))
 (segment (start 195.58 92.71) (end 198.12 96.52) (width 0.25) (layer B.Cu) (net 14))
 (segment (start 189.23 86.36) (end 195.58 92.71) (width 0.25) (layer B.Cu) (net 14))
 (segment (start 189.23 83.82) (end 189.23 86.36) (width 0.25) (layer B.Cu) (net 14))
 (segment (start 172.72 102.87) (end 172.72 104.14) (width 0.25) (layer B.Cu) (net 14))
 (segment (start 189.23 86.36) (end 172.72 102.87) (width 0.25) (layer B.Cu) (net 14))
 (segment (start 198.12 96.52) (end 201.93 100.33) (width 0.25) (layer B.Cu) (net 14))
 (segment (start 170.18 100.33) (end 170.18 104.14) (width 0.25) (layer B.Cu) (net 15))
 (segment (start 186.69 83.82) (end 170.18 100.33) (width 0.25) (layer B.Cu) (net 15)))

